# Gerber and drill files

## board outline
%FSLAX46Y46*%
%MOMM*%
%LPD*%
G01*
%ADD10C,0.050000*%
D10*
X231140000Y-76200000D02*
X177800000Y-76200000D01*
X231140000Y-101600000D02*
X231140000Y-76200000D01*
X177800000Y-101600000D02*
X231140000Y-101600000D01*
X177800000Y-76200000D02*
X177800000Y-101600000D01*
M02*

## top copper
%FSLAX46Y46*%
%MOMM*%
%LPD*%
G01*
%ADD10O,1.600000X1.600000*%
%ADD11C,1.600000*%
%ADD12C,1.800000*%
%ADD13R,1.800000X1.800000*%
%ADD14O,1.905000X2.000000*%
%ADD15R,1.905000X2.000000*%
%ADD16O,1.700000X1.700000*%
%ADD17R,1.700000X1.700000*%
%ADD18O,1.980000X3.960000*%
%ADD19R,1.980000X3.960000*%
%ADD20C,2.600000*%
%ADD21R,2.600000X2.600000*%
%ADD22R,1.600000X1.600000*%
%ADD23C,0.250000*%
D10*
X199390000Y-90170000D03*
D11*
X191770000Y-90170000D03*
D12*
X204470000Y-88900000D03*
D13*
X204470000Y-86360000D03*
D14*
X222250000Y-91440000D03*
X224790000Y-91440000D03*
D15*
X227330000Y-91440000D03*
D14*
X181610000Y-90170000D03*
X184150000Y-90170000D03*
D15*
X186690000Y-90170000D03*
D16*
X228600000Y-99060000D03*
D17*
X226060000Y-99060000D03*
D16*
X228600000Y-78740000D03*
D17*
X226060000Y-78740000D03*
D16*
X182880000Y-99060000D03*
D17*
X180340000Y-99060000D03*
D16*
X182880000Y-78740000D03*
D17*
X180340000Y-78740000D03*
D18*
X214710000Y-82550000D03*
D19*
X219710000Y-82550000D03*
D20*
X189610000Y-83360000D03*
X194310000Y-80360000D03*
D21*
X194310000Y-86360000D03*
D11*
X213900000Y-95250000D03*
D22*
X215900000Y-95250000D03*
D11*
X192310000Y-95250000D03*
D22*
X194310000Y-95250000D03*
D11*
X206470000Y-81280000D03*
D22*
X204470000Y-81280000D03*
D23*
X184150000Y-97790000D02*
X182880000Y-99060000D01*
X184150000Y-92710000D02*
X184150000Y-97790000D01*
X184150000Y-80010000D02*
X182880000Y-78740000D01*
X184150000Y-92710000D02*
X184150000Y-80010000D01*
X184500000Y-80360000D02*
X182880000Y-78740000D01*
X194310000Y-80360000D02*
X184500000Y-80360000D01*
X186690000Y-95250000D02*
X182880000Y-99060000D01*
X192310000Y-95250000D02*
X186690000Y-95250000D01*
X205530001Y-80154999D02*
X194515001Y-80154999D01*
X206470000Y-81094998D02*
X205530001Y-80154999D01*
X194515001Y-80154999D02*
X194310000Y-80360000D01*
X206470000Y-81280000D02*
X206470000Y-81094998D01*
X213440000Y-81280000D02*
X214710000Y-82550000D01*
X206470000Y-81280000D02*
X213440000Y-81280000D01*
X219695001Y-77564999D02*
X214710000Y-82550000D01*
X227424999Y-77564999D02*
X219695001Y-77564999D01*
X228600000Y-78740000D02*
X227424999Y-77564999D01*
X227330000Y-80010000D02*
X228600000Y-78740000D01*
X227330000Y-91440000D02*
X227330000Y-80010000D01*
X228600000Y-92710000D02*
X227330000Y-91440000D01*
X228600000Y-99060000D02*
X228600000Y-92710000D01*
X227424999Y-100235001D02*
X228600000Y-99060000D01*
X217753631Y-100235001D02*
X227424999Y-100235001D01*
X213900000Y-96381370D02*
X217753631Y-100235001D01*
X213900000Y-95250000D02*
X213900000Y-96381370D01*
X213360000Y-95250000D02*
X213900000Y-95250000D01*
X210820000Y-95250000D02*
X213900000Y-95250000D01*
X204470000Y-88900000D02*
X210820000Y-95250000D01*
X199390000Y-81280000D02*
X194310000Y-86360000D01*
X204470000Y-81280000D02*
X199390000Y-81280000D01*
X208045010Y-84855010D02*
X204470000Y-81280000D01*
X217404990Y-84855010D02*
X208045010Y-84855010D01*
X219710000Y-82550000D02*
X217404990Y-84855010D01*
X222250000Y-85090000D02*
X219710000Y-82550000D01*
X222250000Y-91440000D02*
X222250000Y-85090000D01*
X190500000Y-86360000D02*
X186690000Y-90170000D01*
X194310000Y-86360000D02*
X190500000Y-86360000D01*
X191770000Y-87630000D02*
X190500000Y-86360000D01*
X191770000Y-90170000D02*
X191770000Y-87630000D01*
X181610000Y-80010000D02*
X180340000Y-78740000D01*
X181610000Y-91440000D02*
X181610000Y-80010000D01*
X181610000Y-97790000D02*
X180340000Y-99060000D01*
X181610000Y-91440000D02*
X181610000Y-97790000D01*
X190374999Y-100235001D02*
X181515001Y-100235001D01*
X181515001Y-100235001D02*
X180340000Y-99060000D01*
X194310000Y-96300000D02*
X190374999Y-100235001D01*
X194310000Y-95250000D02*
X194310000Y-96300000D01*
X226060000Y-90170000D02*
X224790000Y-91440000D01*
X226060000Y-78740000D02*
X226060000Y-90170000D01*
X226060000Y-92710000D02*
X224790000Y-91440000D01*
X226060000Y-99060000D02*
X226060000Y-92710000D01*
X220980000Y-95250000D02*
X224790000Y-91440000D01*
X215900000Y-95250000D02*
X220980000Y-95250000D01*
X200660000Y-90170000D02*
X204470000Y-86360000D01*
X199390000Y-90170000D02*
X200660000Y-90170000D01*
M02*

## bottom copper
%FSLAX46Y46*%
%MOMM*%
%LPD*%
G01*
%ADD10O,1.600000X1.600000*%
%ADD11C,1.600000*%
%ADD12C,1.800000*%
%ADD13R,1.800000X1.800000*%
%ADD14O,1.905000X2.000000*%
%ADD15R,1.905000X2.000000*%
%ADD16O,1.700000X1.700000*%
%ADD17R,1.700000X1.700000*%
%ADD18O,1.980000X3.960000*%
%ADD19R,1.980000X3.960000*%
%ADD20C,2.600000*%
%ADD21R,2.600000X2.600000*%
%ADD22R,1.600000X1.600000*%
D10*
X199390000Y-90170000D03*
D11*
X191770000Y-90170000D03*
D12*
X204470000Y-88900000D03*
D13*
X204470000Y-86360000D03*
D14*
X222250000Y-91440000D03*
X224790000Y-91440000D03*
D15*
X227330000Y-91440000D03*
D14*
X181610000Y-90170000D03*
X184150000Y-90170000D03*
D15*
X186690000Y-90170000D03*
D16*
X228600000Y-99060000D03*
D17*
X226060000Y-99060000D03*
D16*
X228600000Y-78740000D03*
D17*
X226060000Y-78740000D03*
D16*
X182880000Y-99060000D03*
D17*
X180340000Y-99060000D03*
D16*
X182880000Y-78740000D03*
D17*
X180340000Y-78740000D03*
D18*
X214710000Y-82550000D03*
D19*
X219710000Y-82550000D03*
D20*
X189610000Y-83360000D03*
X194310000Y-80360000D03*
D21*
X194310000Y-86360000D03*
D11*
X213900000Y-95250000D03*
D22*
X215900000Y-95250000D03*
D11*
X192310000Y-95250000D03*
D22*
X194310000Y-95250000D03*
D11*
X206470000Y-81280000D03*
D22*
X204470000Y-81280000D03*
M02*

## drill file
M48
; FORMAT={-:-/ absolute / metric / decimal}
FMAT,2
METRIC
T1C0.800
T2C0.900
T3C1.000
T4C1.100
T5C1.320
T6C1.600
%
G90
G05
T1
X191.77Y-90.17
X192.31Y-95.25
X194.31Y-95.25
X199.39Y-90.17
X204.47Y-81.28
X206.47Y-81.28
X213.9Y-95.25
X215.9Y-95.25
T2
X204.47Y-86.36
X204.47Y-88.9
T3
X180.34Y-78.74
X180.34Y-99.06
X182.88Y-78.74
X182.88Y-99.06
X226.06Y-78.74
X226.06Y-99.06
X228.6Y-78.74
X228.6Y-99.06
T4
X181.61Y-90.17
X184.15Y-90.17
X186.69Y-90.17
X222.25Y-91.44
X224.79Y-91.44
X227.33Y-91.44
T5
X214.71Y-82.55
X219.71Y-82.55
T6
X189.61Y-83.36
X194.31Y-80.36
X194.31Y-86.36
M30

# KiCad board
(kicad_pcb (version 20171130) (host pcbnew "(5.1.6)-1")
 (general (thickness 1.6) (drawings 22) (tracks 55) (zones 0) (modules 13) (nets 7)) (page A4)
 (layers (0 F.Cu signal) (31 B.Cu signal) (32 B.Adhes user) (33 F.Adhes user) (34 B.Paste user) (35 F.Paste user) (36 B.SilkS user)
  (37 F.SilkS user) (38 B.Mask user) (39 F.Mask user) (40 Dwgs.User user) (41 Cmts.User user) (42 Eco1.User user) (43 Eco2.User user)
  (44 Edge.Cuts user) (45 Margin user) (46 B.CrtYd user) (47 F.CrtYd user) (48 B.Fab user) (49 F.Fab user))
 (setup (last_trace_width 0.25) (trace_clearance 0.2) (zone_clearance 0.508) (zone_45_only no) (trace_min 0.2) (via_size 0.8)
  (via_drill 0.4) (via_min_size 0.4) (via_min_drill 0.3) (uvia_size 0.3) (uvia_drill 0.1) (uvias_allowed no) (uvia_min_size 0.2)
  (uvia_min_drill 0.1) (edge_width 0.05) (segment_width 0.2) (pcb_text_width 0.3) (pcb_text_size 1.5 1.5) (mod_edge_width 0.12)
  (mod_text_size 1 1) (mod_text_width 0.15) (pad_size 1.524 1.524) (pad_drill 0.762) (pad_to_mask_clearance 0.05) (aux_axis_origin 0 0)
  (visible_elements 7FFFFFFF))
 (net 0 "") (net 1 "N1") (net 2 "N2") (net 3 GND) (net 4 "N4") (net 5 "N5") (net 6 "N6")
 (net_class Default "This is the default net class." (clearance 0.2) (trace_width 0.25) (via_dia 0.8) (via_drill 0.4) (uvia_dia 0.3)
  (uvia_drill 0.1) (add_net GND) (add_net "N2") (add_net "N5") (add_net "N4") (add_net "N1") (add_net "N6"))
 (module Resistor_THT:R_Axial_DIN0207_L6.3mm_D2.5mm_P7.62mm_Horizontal (layer F.Cu) (at 191.77 90.17)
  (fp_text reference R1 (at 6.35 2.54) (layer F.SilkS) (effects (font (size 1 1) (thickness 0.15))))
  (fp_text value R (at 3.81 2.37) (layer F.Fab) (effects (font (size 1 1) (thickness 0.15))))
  (pad 2 thru_hole oval (at 7.62 0) (size 1.6 1.6) (drill 0.8) (layers *.Cu *.Mask) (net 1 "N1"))
  (pad 1 thru_hole circle (at 0 0) (size 1.6 1.6) (drill 0.8) (layers *.Cu *.Mask) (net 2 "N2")))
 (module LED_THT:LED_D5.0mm (layer F.Cu) (at 204.47 86.36 270)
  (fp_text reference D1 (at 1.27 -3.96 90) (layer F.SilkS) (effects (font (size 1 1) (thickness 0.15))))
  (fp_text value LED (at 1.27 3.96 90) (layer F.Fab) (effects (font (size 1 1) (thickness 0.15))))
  (pad 2 thru_hole circle (at 2.54 0 270) (size 1.8 1.8) (drill 0.9) (layers *.Cu *.Mask) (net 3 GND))
  (pad 1 thru_hole rect (at 0 0 270) (size 1.8 1.8) (drill 0.9) (layers *.Cu *.Mask) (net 1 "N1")))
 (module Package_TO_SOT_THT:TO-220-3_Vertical (layer F.Cu) (at 227.33 91.44 180)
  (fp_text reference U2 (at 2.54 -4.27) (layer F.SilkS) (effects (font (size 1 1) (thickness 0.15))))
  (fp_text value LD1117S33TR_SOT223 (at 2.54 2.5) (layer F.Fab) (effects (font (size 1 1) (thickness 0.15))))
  (pad 3 thru_hole oval (at 5.08 0 180) (size 1.905 2) (drill 1.1) (layers *.Cu *.Mask) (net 2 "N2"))
  (pad 2 thru_hole oval (at 2.54 0 180) (size 1.905 2) (drill 1.1) (layers *.Cu *.Mask) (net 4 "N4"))
  (pad 1 thru_hole rect (at 0 0 180) (size 1.905 2) (drill 1.1) (layers *.Cu *.Mask) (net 3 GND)))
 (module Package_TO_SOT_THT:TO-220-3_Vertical (layer F.Cu) (at 186.69 90.17 180)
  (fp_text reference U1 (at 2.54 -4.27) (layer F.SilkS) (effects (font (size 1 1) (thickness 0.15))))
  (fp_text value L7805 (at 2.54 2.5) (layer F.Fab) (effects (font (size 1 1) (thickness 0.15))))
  (pad 3 thru_hole oval (at 5.08 0 180) (size 1.905 2) (drill 1.1) (layers *.Cu *.Mask) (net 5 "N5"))
  (pad 2 thru_hole oval (at 2.54 0 180) (size 1.905 2) (drill 1.1) (layers *.Cu *.Mask) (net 3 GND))
  (pad 1 thru_hole rect (at 0 0 180) (size 1.905 2) (drill 1.1) (layers *.Cu *.Mask) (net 2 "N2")))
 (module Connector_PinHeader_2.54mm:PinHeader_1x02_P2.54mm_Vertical (layer F.Cu) (at 226.06 99.06 90)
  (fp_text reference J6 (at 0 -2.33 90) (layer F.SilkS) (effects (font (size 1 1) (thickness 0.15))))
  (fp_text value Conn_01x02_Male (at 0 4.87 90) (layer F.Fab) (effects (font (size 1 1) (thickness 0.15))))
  (pad 2 thru_hole oval (at 0 2.54 90) (size 1.7 1.7) (drill 1) (layers *.Cu *.Mask) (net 3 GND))
  (pad 1 thru_hole rect (at 0 0 90) (size 1.7 1.7) (drill 1) (layers *.Cu *.Mask) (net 4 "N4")))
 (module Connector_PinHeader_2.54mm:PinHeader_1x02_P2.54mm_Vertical (layer F.Cu) (at 226.06 78.74 90)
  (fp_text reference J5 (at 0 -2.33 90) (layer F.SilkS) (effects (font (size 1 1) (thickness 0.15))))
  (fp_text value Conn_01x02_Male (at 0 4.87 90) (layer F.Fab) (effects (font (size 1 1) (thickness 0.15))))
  (pad 2 thru_hole oval (at 0 2.54 90) (size 1.7 1.7) (drill 1) (layers *.Cu *.Mask) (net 3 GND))
  (pad 1 thru_hole rect (at 0 0 90) (size 1.7 1.7) (drill 1) (layers *.Cu *.Mask) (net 4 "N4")))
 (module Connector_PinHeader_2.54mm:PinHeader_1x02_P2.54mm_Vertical (layer F.Cu) (at 180.34 99.06 90)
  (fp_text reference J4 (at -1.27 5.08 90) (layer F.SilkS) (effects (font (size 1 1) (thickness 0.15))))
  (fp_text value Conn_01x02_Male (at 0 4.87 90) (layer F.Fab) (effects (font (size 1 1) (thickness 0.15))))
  (pad 2 thru_hole oval (at 0 2.54 90) (size 1.7 1.7) (drill 1) (layers *.Cu *.Mask) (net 3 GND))
  (pad 1 thru_hole rect (at 0 0 90) (size 1.7 1.7) (drill 1) (layers *.Cu *.Mask) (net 5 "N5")))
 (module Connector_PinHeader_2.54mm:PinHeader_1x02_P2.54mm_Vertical (layer F.Cu) (at 180.34 78.74 90)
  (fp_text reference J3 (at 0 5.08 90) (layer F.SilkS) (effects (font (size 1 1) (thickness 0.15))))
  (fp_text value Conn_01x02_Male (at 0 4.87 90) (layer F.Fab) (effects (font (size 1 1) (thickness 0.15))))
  (pad 2 thru_hole oval (at 0 2.54 90) (size 1.7 1.7) (drill 1) (layers *.Cu *.Mask) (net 3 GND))
  (pad 1 thru_hole rect (at 0 0 90) (size 1.7 1.7) (drill 1) (layers *.Cu *.Mask) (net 5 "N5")))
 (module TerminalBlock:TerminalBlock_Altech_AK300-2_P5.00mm (layer F.Cu) (at 219.71 82.55 180)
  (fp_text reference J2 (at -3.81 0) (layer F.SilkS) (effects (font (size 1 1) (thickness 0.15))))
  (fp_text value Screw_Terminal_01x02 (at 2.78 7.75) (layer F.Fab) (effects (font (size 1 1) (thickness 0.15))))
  (pad 2 thru_hole oval (at 5 0 180) (size 1.98 3.96) (drill 1.32) (layers *.Cu *.Mask) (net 3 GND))
  (pad 1 thru_hole rect (at 0 0 180) (size 1.98 3.96) (drill 1.32) (layers *.Cu *.Mask) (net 2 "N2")))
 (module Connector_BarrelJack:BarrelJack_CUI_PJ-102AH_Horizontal (layer F.Cu) (at 194.31 86.36 180)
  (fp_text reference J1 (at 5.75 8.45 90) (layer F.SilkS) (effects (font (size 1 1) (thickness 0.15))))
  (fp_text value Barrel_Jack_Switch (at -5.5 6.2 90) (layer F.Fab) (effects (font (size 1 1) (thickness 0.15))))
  (pad 3 thru_hole circle (at 4.7 3 180) (size 2.6 2.6) (drill 1.6) (layers *.Cu *.Mask) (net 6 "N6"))
  (pad 2 thru_hole circle (at 0 6 180) (size 2.6 2.6) (drill 1.6) (layers *.Cu *.Mask) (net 3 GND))
  (pad 1 thru_hole rect (at 0 0 180) (size 2.6 2.6) (drill 1.6) (layers *.Cu *.Mask) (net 2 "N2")))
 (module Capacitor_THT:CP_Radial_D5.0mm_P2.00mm (layer F.Cu) (at 215.9 95.25 180)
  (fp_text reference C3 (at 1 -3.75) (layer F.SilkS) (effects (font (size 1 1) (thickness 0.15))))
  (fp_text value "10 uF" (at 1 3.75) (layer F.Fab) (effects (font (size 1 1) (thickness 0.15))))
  (pad 2 thru_hole circle (at 2 0 180) (size 1.6 1.6) (drill 0.8) (layers *.Cu *.Mask) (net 3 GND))
  (pad 1 thru_hole rect (at 0 0 180) (size 1.6 1.6) (drill 0.8) (layers *.Cu *.Mask) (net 4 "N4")))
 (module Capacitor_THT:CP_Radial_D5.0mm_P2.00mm (layer F.Cu) (at 194.31 95.25 180)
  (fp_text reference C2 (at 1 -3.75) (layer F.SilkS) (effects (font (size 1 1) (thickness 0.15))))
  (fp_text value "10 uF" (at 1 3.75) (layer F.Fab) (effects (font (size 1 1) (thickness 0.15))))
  (pad 2 thru_hole circle (at 2 0 180) (size 1.6 1.6) (drill 0.8) (layers *.Cu *.Mask) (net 3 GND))
  (pad 1 thru_hole rect (at 0 0 180) (size 1.6 1.6) (drill 0.8) (layers *.Cu *.Mask) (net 5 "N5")))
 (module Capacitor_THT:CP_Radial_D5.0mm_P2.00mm (layer F.Cu) (at 204.47 81.28)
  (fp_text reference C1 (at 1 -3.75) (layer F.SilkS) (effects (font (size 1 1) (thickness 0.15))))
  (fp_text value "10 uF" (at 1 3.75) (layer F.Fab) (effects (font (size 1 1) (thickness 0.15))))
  (pad 2 thru_hole circle (at 2 0) (size 1.6 1.6) (drill 0.8) (layers *.Cu *.Mask) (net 3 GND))
  (pad 1 thru_hole rect (at 0 0) (size 1.6 1.6) (drill 0.8) (layers *.Cu *.Mask) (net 2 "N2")))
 (gr_line (start 231.14 76.2) (end 177.8 76.2) (layer Edge.Cuts) (width 0.05))
 (gr_line (start 231.14 101.6) (end 231.14 76.2) (layer Edge.Cuts) (width 0.05))
 (gr_line (start 177.8 101.6) (end 231.14 101.6) (layer Edge.Cuts) (width 0.05))
 (gr_line (start 177.8 76.2) (end 177.8 101.6) (layer Edge.Cuts) (width 0.05))
 (segment (start 184.15 97.79) (end 182.88 99.06) (width 0.25) (layer F.Cu) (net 3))
 (segment (start 184.15 92.71) (end 184.15 97.79) (width 0.25) (layer F.Cu) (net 3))
 (segment (start 184.15 80.01) (end 182.88 78.74) (width 0.25) (layer F.Cu) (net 3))
 (segment (start 184.15 92.71) (end 184.15 80.01) (width 0.25) (layer F.Cu) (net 3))
 (segment (start 184.5 80.36) (end 182.88 78.74) (width 0.25) (layer F.Cu) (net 3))
 (segment (start 194.31 80.36) (end 184.5 80.36) (width 0.25) (layer F.Cu) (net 3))
 (segment (start 186.69 95.25) (end 182.88 99.06) (width 0.25) (layer F.Cu) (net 3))
 (segment (start 192.31 95.25) (end 186.69 95.25) (width 0.25) (layer F.Cu) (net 3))
 (segment (start 205.530001 80.154999) (end 194.515001 80.154999) (width 0.25) (layer F.Cu) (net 3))
 (segment (start 206.47 81.094998) (end 205.530001 80.154999) (width 0.25) (layer F.Cu) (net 3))
 (segment (start 194.515001 80.154999) (end 194.31 80.36) (width 0.25) (layer F.Cu) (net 3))
 (segment (start 206.47 81.28) (end 206.47 81.094998) (width 0.25) (layer F.Cu) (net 3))
 (segment (start 213.44 81.28) (end 214.71 82.55) (width 0.25) (layer F.Cu) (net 3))
 (segment (start 206.47 81.28) (end 213.44 81.28) (width 0.25) (layer F.Cu) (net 3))
 (segment (start 219.695001 77.564999) (end 214.71 82.55) (width 0.25) (layer F.Cu) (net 3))
 (segment (start 227.424999 77.564999) (end 219.695001 77.564999) (width 0.25) (layer F.Cu) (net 3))
 (segment (start 228.6 78.74) (end 227.424999 77.564999) (width 0.25) (layer F.Cu) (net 3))
 (segment (start 227.33 80.01) (end 228.6 78.74) (width 0.25) (layer F.Cu) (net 3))
 (segment (start 227.33 91.44) (end 227.33 80.01) (width 0.25) (layer F.Cu) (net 3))
 (segment (start 228.6 92.71) (end 227.33 91.44) (width 0.25) (layer F.Cu) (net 3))
 (segment (start 228.6 99.06) (end 228.6 92.71) (width 0.25) (layer F.Cu) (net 3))
 (segment (start 227.424999 100.235001) (end 228.6 99.06) (width 0.25) (layer F.Cu) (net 3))
 (segment (start 217.753631 100.235001) (end 227.424999 100.235001) (width 0.25) (layer F.Cu) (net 3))
 (segment (start 213.9 96.38137) (end 217.753631 100.235001) (width 0.25) (layer F.Cu) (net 3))
 (segment (start 213.9 95.25) (end 213.9 96.38137) (width 0.25) (layer F.Cu) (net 3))
 (segment (start 213.36 95.25) (end 213.9 95.25) (width 0.25) (layer F.Cu) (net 3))
 (segment (start 210.82 95.25) (end 213.9 95.25) (width 0.25) (layer F.Cu) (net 3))
 (segment (start 204.47 88.9) (end 210.82 95.25) (width 0.25) (layer F.Cu) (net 3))
 (segment (start 199.39 81.28) (end 194.31 86.36) (width 0.25) (layer F.Cu) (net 2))
 (segment (start 204.47 81.28) (end 199.39 81.28) (width 0.25) (layer F.Cu) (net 2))
 (segment (start 208.04501 84.85501) (end 204.47 81.28) (width 0.25) (layer F.Cu) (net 2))
 (segment (start 217.40499 84.85501) (end 208.04501 84.85501) (width 0.25) (layer F.Cu) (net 2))
 (segment (start 219.71 82.55) (end 217.40499 84.85501) (width 0.25) (layer F.Cu) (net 2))
 (segment (start 222.25 85.09) (end 219.71 82.55) (width 0.25) (layer F.Cu) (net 2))
 (segment (start 222.25 91.44) (end 222.25 85.09) (width 0.25) (layer F.Cu) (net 2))
 (segment (start 190.5 86.36) (end 186.69 90.17) (width 0.25) (layer F.Cu) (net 2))
 (segment (start 194.31 86.36) (end 190.5 86.36) (width 0.25) (layer F.Cu) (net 2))
 (segment (start 191.77 87.63) (end 190.5 86.36) (width 0.25) (layer F.Cu) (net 2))
 (segment (start 191.77 90.17) (end 191.77 87.63) (width 0.25) (layer F.Cu) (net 2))
 (segment (start 181.61 80.01) (end 180.34 78.74) (width 0.25) (layer F.Cu) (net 5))
 (segment (start 181.61 91.44) (end 181.61 80.01) (width 0.25) (layer F.Cu) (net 5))
 (segment (start 181.61 97.79) (end 180.34 99.06) (width 0.25) (layer F.Cu) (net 5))
 (segment (start 181.61 91.44) (end 181.61 97.79) (width 0.25) (layer F.Cu) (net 5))
 (segment (start 190.374999 100.235001) (end 181.515001 100.235001) (width 0.25) (layer F.Cu) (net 5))
 (segment (start 181.515001 100.235001) (end 180.34 99.06) (width 0.25) (layer F.Cu) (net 5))
 (segment (start 194.31 96.3) (end 190.374999 100.235001) (width 0.25) (layer F.Cu) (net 5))
 (segment (start 194.31 95.25) (end 194.31 96.3) (width 0.25) (layer F.Cu) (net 5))
 (segment (start 226.06 90.17) (end 224.79 91.44) (width 0.25) (layer F.Cu) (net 4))
 (segment (start 226.06 78.74) (end 226.06 90.17) (width 0.25) (layer F.Cu) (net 4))
 (segment (start 226.06 92.71) (end 224.79 91.44) (width 0.25) (layer F.Cu) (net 4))
 (segment (start 226.06 99.06) (end 226.06 92.71) (width 0.25) (layer F.Cu) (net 4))
 (segment (start 220.98 95.25) (end 224.79 91.44) (width 0.25) (layer F.Cu) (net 4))
 (segment (start 215.9 95.25) (end 220.98 95.25) (width 0.25) (layer F.Cu) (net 4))
 (segment (start 200.66 90.17) (end 204.47 86.36) (width 0.25) (layer F.Cu) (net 1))
 (segment (start 199.39 90.17) (end 200.66 90.17) (width 0.25) (layer F.Cu) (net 1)))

